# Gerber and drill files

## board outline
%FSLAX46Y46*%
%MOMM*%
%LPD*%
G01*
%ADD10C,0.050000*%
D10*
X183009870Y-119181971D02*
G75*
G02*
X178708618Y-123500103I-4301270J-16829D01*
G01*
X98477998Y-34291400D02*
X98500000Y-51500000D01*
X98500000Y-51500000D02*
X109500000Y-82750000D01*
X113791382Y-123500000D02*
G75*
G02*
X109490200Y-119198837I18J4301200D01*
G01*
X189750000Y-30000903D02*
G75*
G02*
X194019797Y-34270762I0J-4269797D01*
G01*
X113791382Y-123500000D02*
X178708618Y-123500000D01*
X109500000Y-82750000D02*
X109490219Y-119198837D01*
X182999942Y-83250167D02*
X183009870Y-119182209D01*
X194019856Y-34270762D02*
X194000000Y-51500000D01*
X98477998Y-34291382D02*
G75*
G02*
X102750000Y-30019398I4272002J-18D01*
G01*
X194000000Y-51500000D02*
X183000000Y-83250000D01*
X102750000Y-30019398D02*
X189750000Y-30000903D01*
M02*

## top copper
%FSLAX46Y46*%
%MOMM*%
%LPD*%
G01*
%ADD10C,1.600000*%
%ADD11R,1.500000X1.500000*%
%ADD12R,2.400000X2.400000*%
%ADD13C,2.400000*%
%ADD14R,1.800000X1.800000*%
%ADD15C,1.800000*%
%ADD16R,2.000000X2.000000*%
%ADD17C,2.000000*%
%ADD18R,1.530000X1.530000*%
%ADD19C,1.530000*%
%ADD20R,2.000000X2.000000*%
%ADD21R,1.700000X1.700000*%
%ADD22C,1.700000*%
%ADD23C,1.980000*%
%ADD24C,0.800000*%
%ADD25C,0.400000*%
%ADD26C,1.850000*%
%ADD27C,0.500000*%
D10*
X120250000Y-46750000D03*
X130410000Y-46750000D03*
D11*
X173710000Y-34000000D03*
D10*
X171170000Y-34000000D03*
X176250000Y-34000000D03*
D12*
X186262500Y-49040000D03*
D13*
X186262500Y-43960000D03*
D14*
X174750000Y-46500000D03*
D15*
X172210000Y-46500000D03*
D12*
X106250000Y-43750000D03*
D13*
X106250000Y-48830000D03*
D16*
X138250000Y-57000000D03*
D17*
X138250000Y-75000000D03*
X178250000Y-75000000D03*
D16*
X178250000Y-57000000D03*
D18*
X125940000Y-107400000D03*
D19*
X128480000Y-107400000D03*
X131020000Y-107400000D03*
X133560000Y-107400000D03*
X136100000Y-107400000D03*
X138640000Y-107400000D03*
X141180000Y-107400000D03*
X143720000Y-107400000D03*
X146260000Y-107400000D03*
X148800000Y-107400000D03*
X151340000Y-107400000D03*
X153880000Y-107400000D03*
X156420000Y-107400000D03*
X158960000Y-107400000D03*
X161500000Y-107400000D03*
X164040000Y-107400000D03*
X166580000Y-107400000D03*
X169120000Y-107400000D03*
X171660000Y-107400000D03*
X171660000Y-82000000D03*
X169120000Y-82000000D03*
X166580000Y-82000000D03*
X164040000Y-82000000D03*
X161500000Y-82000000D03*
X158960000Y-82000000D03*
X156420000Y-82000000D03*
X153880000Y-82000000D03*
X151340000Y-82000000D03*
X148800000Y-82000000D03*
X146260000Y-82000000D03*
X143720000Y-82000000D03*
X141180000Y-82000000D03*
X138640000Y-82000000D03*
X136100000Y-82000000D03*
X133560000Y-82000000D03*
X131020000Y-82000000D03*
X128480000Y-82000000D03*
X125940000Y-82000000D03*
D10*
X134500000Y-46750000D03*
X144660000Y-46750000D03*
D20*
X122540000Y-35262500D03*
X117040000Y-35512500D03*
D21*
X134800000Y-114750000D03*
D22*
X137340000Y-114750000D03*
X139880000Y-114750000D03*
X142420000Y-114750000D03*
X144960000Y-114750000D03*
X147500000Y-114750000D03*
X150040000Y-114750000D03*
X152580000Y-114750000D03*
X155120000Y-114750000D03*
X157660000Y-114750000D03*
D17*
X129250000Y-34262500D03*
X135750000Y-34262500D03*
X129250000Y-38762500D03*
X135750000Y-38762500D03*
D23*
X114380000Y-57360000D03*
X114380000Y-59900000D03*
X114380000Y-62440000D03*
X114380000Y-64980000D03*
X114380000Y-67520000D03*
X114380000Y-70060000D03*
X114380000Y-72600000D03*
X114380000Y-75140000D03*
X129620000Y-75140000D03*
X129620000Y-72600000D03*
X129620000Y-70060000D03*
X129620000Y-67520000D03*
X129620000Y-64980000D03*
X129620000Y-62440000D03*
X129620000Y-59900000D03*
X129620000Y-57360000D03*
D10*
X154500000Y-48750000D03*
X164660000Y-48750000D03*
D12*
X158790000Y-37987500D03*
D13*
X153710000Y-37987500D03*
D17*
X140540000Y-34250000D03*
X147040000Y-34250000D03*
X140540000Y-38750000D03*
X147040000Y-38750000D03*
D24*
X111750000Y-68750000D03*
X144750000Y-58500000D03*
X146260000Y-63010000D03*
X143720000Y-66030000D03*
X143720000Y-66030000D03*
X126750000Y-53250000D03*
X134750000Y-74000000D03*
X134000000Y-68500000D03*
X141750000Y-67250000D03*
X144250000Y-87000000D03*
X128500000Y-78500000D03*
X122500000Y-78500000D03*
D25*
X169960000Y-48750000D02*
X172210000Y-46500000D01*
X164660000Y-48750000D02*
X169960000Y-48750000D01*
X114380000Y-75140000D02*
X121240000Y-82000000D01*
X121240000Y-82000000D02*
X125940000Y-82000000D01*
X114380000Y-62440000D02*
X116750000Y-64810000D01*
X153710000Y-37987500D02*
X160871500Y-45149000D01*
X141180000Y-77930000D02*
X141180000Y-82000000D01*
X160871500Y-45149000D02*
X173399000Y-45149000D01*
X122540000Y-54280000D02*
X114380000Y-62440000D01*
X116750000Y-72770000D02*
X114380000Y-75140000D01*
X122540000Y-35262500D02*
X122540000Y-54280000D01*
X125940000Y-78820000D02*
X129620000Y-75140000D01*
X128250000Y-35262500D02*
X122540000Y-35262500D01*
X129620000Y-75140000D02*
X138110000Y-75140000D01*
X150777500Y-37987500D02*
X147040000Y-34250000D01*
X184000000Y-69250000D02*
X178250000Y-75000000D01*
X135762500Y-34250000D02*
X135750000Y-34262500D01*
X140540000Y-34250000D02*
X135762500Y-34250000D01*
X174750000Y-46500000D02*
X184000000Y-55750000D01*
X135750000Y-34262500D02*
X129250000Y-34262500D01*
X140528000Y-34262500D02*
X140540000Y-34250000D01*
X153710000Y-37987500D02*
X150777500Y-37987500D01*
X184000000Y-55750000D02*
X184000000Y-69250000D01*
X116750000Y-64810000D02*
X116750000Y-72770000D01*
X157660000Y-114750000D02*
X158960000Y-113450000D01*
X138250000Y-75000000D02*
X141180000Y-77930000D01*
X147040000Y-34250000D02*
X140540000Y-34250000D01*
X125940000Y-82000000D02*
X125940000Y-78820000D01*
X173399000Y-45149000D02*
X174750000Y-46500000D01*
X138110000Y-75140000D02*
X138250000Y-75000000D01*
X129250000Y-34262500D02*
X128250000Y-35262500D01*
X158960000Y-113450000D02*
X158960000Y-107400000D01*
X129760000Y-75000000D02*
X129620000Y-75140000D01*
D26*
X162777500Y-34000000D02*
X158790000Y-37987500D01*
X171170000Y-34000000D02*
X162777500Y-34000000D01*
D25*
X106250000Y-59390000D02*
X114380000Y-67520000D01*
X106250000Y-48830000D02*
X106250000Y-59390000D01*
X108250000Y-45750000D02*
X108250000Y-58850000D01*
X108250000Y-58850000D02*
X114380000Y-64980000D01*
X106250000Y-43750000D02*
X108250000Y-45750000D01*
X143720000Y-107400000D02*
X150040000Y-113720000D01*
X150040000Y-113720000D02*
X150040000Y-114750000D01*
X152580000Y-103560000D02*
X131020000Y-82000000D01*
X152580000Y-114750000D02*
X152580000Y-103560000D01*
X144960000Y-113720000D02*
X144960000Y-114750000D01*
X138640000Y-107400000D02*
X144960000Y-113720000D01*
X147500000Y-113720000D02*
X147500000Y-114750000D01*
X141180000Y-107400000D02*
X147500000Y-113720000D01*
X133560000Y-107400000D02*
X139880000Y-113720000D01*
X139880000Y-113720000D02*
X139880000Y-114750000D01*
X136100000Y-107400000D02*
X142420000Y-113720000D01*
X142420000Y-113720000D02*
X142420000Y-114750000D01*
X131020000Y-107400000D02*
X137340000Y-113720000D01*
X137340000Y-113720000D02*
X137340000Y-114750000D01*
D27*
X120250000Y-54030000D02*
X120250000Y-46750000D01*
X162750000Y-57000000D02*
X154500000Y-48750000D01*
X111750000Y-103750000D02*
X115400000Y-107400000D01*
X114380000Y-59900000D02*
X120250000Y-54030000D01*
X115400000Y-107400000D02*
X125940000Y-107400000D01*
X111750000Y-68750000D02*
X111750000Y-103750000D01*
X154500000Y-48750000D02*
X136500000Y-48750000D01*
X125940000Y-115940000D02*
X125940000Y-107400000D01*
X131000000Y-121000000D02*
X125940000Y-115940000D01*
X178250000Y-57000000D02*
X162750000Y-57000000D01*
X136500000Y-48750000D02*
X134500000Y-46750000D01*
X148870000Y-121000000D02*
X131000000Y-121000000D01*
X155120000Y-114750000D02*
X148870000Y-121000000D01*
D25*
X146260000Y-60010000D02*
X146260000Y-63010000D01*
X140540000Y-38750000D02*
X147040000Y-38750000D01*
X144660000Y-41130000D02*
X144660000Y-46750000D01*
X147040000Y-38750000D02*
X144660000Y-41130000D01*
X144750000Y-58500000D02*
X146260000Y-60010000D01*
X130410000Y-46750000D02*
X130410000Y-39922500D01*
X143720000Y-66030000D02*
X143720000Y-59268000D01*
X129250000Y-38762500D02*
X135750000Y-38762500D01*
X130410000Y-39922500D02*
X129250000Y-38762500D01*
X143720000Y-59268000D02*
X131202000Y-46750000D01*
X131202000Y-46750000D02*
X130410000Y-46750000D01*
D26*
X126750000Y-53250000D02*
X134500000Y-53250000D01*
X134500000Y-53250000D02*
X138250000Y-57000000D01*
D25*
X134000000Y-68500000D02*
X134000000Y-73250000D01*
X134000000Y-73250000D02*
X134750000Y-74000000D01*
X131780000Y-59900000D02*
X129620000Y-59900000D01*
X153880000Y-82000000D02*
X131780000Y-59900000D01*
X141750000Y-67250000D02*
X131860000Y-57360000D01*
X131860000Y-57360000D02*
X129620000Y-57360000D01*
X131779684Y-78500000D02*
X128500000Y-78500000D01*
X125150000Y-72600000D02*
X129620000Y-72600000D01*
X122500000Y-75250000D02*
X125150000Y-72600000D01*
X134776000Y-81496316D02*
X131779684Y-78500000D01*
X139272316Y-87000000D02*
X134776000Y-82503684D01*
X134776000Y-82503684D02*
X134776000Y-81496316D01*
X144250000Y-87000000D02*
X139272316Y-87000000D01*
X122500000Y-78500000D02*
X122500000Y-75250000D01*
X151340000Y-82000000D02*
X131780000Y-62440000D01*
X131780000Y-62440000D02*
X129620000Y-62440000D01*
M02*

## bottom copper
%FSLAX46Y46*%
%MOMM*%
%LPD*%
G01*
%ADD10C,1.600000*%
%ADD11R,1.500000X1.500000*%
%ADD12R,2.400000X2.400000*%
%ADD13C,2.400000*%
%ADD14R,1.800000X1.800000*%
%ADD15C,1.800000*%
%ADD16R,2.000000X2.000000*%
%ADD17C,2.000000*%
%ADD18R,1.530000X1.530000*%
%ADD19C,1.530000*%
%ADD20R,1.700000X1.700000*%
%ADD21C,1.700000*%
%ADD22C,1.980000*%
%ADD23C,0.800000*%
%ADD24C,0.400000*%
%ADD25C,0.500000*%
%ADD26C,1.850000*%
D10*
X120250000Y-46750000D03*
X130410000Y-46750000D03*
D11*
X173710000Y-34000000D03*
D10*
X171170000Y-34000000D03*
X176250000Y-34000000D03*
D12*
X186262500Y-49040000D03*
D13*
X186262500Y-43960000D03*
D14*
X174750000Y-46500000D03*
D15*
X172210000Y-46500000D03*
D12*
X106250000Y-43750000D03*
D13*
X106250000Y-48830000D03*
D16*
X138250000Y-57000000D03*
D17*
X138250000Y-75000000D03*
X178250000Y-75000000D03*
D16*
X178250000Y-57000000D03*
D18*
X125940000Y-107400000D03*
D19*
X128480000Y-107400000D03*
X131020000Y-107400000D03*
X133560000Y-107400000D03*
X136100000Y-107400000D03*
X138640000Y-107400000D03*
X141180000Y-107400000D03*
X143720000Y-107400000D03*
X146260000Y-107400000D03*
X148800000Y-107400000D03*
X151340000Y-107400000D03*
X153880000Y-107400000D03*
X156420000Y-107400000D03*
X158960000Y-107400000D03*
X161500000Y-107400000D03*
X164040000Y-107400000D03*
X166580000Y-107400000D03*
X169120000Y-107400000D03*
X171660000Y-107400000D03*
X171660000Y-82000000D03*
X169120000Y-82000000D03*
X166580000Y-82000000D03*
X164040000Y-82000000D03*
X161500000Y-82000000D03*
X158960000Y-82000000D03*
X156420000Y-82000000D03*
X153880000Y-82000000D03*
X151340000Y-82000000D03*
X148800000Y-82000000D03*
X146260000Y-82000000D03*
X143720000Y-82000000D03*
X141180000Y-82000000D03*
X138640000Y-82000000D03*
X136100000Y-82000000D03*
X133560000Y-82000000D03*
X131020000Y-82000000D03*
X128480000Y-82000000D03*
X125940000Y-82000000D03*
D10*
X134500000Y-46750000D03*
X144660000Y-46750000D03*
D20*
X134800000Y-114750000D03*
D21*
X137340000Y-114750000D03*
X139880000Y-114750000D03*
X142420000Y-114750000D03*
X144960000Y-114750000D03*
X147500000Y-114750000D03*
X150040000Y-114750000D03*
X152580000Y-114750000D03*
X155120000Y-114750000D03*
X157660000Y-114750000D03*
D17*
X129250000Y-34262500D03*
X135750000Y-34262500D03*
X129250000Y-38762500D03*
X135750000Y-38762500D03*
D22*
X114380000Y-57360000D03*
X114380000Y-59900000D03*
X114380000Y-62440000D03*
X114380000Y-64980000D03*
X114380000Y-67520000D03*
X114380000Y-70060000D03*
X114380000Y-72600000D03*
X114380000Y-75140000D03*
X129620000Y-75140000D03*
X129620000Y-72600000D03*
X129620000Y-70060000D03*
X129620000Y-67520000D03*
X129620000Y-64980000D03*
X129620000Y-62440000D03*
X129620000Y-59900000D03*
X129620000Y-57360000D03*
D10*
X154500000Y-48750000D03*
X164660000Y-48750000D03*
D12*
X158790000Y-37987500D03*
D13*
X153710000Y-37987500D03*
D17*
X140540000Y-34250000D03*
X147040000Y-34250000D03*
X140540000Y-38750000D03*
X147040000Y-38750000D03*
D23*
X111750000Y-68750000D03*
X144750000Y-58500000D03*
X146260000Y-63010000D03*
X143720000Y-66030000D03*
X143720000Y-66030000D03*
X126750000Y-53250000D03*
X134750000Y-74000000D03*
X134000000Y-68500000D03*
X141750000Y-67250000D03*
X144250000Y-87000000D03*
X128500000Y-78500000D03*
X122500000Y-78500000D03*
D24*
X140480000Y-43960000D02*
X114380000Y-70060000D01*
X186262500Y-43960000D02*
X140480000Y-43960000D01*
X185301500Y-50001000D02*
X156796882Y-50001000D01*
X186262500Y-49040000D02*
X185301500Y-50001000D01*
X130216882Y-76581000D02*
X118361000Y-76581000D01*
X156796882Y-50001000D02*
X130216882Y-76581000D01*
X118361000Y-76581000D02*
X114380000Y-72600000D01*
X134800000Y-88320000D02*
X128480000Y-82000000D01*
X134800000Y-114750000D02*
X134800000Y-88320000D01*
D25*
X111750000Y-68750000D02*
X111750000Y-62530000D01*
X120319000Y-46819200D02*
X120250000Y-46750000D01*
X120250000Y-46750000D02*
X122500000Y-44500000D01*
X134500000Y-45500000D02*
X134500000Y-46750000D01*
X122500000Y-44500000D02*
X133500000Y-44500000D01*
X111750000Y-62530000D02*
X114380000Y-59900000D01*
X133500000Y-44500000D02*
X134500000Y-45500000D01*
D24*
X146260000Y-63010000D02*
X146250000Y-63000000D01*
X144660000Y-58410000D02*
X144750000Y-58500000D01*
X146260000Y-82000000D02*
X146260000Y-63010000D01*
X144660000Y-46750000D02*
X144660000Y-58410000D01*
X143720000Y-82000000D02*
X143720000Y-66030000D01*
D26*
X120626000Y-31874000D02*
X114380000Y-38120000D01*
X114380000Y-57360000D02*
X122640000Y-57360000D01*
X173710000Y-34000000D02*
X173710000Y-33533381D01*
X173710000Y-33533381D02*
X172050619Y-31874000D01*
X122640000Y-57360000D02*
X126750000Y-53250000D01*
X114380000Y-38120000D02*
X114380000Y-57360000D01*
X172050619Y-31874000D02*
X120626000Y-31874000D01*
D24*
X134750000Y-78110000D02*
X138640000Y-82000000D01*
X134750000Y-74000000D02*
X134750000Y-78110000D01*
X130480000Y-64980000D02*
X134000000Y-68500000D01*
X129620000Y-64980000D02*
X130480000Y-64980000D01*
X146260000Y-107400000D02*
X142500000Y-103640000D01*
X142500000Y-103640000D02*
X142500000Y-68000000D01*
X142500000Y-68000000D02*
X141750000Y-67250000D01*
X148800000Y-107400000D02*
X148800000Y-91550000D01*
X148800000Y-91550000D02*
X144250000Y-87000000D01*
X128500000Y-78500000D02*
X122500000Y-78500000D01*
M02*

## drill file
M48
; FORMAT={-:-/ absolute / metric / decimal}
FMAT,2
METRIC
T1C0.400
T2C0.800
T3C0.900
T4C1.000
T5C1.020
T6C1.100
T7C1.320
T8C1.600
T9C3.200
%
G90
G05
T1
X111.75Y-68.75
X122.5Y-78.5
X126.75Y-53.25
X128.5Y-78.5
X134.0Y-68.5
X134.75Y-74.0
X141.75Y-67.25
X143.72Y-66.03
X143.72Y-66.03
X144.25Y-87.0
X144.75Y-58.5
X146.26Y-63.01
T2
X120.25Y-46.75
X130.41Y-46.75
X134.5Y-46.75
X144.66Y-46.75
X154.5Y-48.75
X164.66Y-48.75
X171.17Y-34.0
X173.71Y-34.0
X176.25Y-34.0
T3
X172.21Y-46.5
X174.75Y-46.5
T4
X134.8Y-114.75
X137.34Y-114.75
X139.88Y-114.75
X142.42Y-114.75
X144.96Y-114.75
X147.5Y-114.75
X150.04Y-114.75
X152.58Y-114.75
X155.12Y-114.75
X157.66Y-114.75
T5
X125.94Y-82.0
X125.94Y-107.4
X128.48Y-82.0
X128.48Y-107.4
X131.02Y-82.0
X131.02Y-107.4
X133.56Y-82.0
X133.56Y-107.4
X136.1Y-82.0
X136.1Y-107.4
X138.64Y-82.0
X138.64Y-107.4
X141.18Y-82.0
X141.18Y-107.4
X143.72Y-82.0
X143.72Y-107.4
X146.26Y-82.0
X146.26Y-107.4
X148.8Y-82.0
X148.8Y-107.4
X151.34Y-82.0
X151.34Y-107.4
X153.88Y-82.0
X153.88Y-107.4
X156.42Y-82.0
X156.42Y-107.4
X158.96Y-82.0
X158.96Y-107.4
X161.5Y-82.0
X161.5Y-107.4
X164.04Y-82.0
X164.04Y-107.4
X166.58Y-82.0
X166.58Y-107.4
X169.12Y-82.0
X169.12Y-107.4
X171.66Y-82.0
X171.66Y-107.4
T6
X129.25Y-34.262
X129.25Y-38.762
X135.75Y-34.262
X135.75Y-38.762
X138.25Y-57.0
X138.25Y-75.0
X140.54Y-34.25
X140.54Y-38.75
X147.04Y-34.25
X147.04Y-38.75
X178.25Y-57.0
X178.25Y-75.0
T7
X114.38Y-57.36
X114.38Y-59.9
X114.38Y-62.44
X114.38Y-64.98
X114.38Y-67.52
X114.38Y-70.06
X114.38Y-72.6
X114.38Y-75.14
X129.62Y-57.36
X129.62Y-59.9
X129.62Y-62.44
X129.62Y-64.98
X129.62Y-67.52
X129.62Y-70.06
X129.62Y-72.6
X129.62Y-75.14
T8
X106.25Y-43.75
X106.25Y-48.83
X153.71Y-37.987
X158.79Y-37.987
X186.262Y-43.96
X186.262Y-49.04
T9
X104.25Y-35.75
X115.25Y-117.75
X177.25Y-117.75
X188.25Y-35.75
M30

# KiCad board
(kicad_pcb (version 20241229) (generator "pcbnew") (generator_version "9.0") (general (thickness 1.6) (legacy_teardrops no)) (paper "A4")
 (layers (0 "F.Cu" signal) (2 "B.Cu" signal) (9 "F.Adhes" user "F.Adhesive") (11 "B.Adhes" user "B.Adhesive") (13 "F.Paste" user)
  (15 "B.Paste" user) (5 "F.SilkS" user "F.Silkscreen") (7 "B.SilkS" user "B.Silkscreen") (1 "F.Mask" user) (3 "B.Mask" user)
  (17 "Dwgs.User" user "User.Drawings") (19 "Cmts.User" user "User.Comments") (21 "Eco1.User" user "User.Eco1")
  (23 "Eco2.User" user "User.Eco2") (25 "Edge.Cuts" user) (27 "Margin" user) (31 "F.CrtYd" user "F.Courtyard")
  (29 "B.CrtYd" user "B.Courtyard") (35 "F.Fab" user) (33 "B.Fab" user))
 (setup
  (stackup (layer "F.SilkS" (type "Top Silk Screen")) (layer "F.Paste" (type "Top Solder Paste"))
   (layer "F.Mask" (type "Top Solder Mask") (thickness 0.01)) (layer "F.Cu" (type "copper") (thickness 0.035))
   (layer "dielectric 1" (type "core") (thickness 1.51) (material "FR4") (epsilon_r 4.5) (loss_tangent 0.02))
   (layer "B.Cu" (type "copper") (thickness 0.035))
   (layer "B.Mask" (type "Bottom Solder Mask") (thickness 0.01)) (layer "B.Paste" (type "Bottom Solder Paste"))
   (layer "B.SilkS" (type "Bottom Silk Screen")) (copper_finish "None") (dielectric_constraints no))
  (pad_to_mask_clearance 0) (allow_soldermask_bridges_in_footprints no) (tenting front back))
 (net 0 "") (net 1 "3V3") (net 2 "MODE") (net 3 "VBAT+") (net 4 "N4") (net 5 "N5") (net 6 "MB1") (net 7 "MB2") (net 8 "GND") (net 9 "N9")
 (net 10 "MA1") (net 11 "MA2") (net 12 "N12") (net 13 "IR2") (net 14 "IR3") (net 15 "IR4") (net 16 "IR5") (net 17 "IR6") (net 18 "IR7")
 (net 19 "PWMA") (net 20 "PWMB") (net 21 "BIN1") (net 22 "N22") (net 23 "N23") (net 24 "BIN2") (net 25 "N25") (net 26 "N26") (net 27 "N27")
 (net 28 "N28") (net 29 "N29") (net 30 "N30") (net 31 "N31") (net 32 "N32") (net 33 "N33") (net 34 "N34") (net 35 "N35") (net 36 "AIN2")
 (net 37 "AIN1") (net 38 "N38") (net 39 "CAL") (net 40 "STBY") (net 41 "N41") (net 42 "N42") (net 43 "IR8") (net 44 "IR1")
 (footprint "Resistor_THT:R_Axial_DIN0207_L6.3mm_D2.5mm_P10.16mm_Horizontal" (layer "F.Cu") (at 120.25 46.75)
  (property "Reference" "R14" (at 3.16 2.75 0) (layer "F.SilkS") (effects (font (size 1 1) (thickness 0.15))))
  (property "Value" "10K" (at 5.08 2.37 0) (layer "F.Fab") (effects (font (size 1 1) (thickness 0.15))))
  (pad "1" thru_hole circle (at 0 0) (size 1.6 1.6) (drill 0.8) (layers "*.Cu" "*.Mask") (remove_unused_layers no) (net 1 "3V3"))
  (pad "2" thru_hole circle (at 10.16 0) (size 1.6 1.6) (drill 0.8) (layers "*.Cu" "*.Mask") (remove_unused_layers no) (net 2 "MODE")))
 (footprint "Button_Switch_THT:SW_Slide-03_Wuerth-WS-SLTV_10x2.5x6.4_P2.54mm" (layer "F.Cu") (at 173.71 34)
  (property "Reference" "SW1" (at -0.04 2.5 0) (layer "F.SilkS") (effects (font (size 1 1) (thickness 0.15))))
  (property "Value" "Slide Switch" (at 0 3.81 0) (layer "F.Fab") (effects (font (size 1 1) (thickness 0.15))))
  (pad "1" thru_hole rect (at 0 0) (size 1.5 1.5) (drill 0.8) (layers "*.Cu" "*.Mask") (remove_unused_layers no) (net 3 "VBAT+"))
  (pad "2" thru_hole circle (at -2.54 0) (size 1.6 1.6) (drill 0.8) (layers "*.Cu" "*.Mask") (remove_unused_layers no) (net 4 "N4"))
  (pad "3" thru_hole circle (at 2.54 0) (size 1.6 1.6) (drill 0.8) (layers "*.Cu" "*.Mask") (remove_unused_layers no) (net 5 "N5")))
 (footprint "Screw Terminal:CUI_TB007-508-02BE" (layer "F.Cu") (at 186.2625 49.04 90)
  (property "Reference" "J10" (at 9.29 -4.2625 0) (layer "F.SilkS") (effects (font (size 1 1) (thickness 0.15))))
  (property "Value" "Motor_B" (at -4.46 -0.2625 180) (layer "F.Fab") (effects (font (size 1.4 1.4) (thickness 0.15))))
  (pad "1" thru_hole rect (at 0 0 90) (size 2.4 2.4) (drill 1.6) (layers "*.Cu" "*.Mask") (remove_unused_layers no) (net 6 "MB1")
   (solder_mask_margin 0.102))
  (pad "2" thru_hole circle (at 5.08 0 90) (size 2.4 2.4) (drill 1.6) (layers "*.Cu" "*.Mask") (remove_unused_layers no) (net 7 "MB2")
   (solder_mask_margin 0.102)))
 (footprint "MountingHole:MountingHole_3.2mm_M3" (layer "F.Cu") (at 177.25 117.75)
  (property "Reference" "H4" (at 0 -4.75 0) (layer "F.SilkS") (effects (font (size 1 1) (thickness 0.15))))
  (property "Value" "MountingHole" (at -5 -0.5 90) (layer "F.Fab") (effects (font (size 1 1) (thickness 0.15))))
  (pad "" np_thru_hole circle (at 0 0) (size 3.2 3.2) (drill 3.2) (layers "*.Cu" "*.Mask")))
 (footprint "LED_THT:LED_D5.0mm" (layer "F.Cu") (at 174.75 46.5 180)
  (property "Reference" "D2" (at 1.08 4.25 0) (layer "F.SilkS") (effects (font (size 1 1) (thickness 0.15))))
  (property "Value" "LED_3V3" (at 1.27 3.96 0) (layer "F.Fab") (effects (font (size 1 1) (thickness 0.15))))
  (pad "1" thru_hole rect (at 0 0 180) (size 1.8 1.8) (drill 0.9) (layers "*.Cu" "*.Mask") (remove_unused_layers no) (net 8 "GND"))
  (pad "2" thru_hole circle (at 2.54 0 180) (size 1.8 1.8) (drill 0.9) (layers "*.Cu" "*.Mask") (remove_unused_layers no) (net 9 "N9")))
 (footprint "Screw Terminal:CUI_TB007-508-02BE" (layer "F.Cu") (at 106.25 43.75 -90)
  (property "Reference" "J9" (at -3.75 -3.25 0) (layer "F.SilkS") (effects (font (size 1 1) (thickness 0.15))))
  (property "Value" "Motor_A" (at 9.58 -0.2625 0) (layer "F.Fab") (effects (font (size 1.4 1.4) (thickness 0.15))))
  (pad "1" thru_hole rect (at 0 0 270) (size 2.4 2.4) (drill 1.6) (layers "*.Cu" "*.Mask") (remove_unused_layers no) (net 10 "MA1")
   (solder_mask_margin 0.102))
  (pad "2" thru_hole circle (at 5.08 0 270) (size 2.4 2.4) (drill 1.6) (layers "*.Cu" "*.Mask") (remove_unused_layers no) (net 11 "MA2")
   (solder_mask_margin 0.102)))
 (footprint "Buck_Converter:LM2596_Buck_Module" (layer "F.Cu") (at 136.85 76.4)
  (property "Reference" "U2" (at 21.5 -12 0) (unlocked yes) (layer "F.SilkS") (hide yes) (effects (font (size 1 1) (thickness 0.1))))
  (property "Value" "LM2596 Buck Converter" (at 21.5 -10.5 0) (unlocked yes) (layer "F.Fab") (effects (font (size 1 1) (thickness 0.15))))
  (pad "1" thru_hole rect (at 1.4 -19.4) (size 2 2) (drill 1.1) (layers "*.Cu" "*.Mask") (remove_unused_layers no) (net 3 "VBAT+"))
  (pad "2" thru_hole circle (at 1.4 -1.4) (size 2 2) (drill 1.1) (layers "*.Cu" "*.Mask") (remove_unused_layers no) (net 8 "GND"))
  (pad "3" thru_hole circle (at 41.4 -1.4) (size 2 2) (drill 1.1) (layers "*.Cu" "*.Mask") (remove_unused_layers no) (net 8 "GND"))
  (pad "4" thru_hole rect (at 41.4 -19.4) (size 2 2) (drill 1.1) (layers "*.Cu" "*.Mask") (remove_unused_layers no) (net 1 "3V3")))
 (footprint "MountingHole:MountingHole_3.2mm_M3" (layer "F.Cu") (at 115.25 117.75)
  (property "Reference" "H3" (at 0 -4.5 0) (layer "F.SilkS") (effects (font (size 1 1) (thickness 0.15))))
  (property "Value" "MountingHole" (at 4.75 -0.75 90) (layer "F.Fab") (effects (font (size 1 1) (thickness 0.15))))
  (pad "" np_thru_hole circle (at 0 0) (size 3.2 3.2) (drill 3.2) (layers "*.Cu" "*.Mask")))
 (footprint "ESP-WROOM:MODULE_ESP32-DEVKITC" (layer "F.Cu") (at 148.79 94.7 90)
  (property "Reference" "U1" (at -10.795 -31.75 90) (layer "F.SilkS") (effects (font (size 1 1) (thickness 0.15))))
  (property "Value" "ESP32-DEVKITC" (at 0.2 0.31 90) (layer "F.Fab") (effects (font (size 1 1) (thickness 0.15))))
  (pad "1" thru_hole rect (at -12.7 -22.85 90) (size 1.53 1.53) (drill 1.02) (layers "*.Cu" "*.Mask") (remove_unused_layers no)
   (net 1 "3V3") (solder_mask_margin 0.102))
  (pad "2" thru_hole circle (at -12.7 -20.31 90) (size 1.53 1.53) (drill 1.02) (layers "*.Cu" "*.Mask") (remove_unused_layers no)
   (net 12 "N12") (solder_mask_margin 0.102))
  (pad "3" thru_hole circle (at -12.7 -17.77 90) (size 1.53 1.53) (drill 1.02) (layers "*.Cu" "*.Mask") (remove_unused_layers no)
   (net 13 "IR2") (solder_mask_margin 0.102))
  (pad "4" thru_hole circle (at -12.7 -15.23 90) (size 1.53 1.53) (drill 1.02) (layers "*.Cu" "*.Mask") (remove_unused_layers no)
   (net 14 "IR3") (solder_mask_margin 0.102))
  (pad "5" thru_hole circle (at -12.7 -12.69 90) (size 1.53 1.53) (drill 1.02) (layers "*.Cu" "*.Mask") (remove_unused_layers no)
   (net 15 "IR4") (solder_mask_margin 0.102))
  (pad "6" thru_hole circle (at -12.7 -10.15 90) (size 1.53 1.53) (drill 1.02) (layers "*.Cu" "*.Mask") (remove_unused_layers no)
   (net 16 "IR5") (solder_mask_margin 0.102))
  (pad "7" thru_hole circle (at -12.7 -7.61 90) (size 1.53 1.53) (drill 1.02) (layers "*.Cu" "*.Mask") (remove_unused_layers no)
   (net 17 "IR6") (solder_mask_margin 0.102))
  (pad "8" thru_hole circle (at -12.7 -5.07 90) (size 1.53 1.53) (drill 1.02) (layers "*.Cu" "*.Mask") (remove_unused_layers no)
   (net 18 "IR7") (solder_mask_margin 0.102))
  (pad "9" thru_hole circle (at -12.7 -2.53 90) (size 1.53 1.53) (drill 1.02) (layers "*.Cu" "*.Mask") (remove_unused_layers no)
   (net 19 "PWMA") (solder_mask_margin 0.102))
  (pad "10" thru_hole circle (at -12.7 0.01 90) (size 1.53 1.53) (drill 1.02) (layers "*.Cu" "*.Mask") (remove_unused_layers no)
   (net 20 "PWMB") (solder_mask_margin 0.102))
  (pad "11" thru_hole circle (at -12.7 2.55 90) (size 1.53 1.53) (drill 1.02) (layers "*.Cu" "*.Mask") (remove_unused_layers no)
   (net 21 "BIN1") (solder_mask_margin 0.102))
  (pad "12" thru_hole circle (at -12.7 5.09 90) (size 1.53 1.53) (drill 1.02) (layers "*.Cu" "*.Mask") (remove_unused_layers no)
   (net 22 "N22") (solder_mask_margin 0.102))
  (pad "13" thru_hole circle (at -12.7 7.63 90) (size 1.53 1.53) (drill 1.02) (layers "*.Cu" "*.Mask") (remove_unused_layers no)
   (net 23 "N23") (solder_mask_margin 0.102))
  (pad "14" thru_hole circle (at -12.7 10.17 90) (size 1.53 1.53) (drill 1.02) (layers "*.Cu" "*.Mask") (remove_unused_layers no)
   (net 8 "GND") (solder_mask_margin 0.102))
  (pad "15" thru_hole circle (at -12.7 12.71 90) (size 1.53 1.53) (drill 1.02) (layers "*.Cu" "*.Mask") (remove_unused_layers no)
   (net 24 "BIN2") (solder_mask_margin 0.102))
  (pad "16" thru_hole circle (at -12.7 15.25 90) (size 1.53 1.53) (drill 1.02) (layers "*.Cu" "*.Mask") (remove_unused_layers no)
   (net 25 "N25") (solder_mask_margin 0.102))
  (pad "17" thru_hole circle (at -12.7 17.79 90) (size 1.53 1.53) (drill 1.02) (layers "*.Cu" "*.Mask") (remove_unused_layers no)
   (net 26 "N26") (solder_mask_margin 0.102))
  (pad "18" thru_hole circle (at -12.7 20.33 90) (size 1.53 1.53) (drill 1.02) (layers "*.Cu" "*.Mask") (remove_unused_layers no)
   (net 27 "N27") (solder_mask_margin 0.102))
  (pad "19" thru_hole circle (at -12.7 22.87 90) (size 1.53 1.53) (drill 1.02) (layers "*.Cu" "*.Mask") (remove_unused_layers no)
   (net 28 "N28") (solder_mask_margin 0.102))
  (pad "20" thru_hole circle (at 12.7 22.87 90) (size 1.53 1.53) (drill 1.02) (layers "*.Cu" "*.Mask") (remove_unused_layers no)
   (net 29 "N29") (solder_mask_margin 0.102))
  (pad "21" thru_hole circle (at 12.7 20.33 90) (size 1.53 1.53) (drill 1.02) (layers "*.Cu" "*.Mask") (remove_unused_layers no)
   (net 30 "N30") (solder_mask_margin 0.102))
  (pad "22" thru_hole circle (at 12.7 17.79 90) (size 1.53 1.53) (drill 1.02) (layers "*.Cu" "*.Mask") (remove_unused_layers no)
   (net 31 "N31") (solder_mask_margin 0.102))
  (pad "23" thru_hole circle (at 12.7 15.25 90) (size 1.53 1.53) (drill 1.02) (layers "*.Cu" "*.Mask") (remove_unused_layers no)
   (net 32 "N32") (solder_mask_margin 0.102))
  (pad "24" thru_hole circle (at 12.7 12.71 90) (size 1.53 1.53) (drill 1.02) (layers "*.Cu" "*.Mask") (remove_unused_layers no)
   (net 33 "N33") (solder_mask_margin 0.102))
  (pad "25" thru_hole circle (at 12.7 10.17 90) (size 1.53 1.53) (drill 1.02) (layers "*.Cu" "*.Mask") (remove_unused_layers no)
   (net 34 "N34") (solder_mask_margin 0.102))
  (pad "26" thru_hole circle (at 12.7 7.63 90) (size 1.53 1.53) (drill 1.02) (layers "*.Cu" "*.Mask") (remove_unused_layers no)
   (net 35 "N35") (solder_mask_margin 0.102))
  (pad "27" thru_hole circle (at 12.7 5.09 90) (size 1.53 1.53) (drill 1.02) (layers "*.Cu" "*.Mask") (remove_unused_layers no)
   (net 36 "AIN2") (solder_mask_margin 0.102))
  (pad "28" thru_hole circle (at 12.7 2.55 90) (size 1.53 1.53) (drill 1.02) (layers "*.Cu" "*.Mask") (remove_unused_layers no)
   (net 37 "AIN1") (solder_mask_margin 0.102))
  (pad "29" thru_hole circle (at 12.7 0.01 90) (size 1.53 1.53) (drill 1.02) (layers "*.Cu" "*.Mask") (remove_unused_layers no)
   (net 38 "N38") (solder_mask_margin 0.102))
  (pad "30" thru_hole circle (at 12.7 -2.53 90) (size 1.53 1.53) (drill 1.02) (layers "*.Cu" "*.Mask") (remove_unused_layers no)
   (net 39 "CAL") (solder_mask_margin 0.102))
  (pad "31" thru_hole circle (at 12.7 -5.07 90) (size 1.53 1.53) (drill 1.02) (layers "*.Cu" "*.Mask") (remove_unused_layers no)
   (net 2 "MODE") (solder_mask_margin 0.102))
  (pad "32" thru_hole circle (at 12.7 -7.61 90) (size 1.53 1.53) (drill 1.02) (layers "*.Cu" "*.Mask") (remove_unused_layers no)
   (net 8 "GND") (solder_mask_margin 0.102))
  (pad "33" thru_hole circle (at 12.7 -10.15 90) (size 1.53 1.53) (drill 1.02) (layers "*.Cu" "*.Mask") (remove_unused_layers no)
   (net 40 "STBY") (solder_mask_margin 0.102))
  (pad "34" thru_hole circle (at 12.7 -12.69 90) (size 1.53 1.53) (drill 1.02) (layers "*.Cu" "*.Mask") (remove_unused_layers no)
   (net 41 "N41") (solder_mask_margin 0.102))
  (pad "35" thru_hole circle (at 12.7 -15.23 90) (size 1.53 1.53) (drill 1.02) (layers "*.Cu" "*.Mask") (remove_unused_layers no)
   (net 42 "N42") (solder_mask_margin 0.102))
  (pad "36" thru_hole circle (at 12.7 -17.77 90) (size 1.53 1.53) (drill 1.02) (layers "*.Cu" "*.Mask") (remove_unused_layers no)
   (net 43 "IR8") (solder_mask_margin 0.102))
  (pad "37" thru_hole circle (at 12.7 -20.31 90) (size 1.53 1.53) (drill 1.02) (layers "*.Cu" "*.Mask") (remove_unused_layers no)
   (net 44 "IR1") (solder_mask_margin 0.102))
  (pad "38" thru_hole circle (at 12.7 -22.85 90) (size 1.53 1.53) (drill 1.02) (layers "*.Cu" "*.Mask") (remove_unused_layers no)
   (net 8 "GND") (solder_mask_margin 0.102)))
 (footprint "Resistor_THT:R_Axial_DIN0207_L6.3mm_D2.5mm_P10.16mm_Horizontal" (layer "F.Cu") (at 134.5 46.75)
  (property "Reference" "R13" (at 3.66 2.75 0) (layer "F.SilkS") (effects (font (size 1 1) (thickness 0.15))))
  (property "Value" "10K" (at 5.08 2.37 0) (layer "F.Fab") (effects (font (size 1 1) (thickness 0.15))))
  (pad "1" thru_hole circle (at 0 0) (size 1.6 1.6) (drill 0.8) (layers "*.Cu" "*.Mask") (remove_unused_layers no) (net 1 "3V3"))
  (pad "2" thru_hole circle (at 10.16 0) (size 1.6 1.6) (drill 0.8) (layers "*.Cu" "*.Mask") (remove_unused_layers no) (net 39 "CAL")))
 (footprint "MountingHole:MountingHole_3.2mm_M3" (layer "F.Cu") (at 188.25 35.75)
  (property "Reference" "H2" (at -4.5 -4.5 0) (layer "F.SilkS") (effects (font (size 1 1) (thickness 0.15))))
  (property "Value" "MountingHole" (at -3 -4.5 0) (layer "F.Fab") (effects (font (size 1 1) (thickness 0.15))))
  (pad "" np_thru_hole circle (at 0 0) (size 3.2 3.2) (drill 3.2) (layers "*.Cu" "*.Mask")))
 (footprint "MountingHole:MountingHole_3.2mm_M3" (layer "F.Cu") (at 104.25 35.75)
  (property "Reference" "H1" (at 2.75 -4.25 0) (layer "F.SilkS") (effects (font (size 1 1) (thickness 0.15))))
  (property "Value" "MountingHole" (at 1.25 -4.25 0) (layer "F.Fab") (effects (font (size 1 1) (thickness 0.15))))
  (pad "" np_thru_hole circle (at 0 0) (size 3.2 3.2) (drill 3.2) (layers "*.Cu" "*.Mask")))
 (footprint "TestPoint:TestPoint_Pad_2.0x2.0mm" (layer "F.Cu") (at 122.54 35.2625)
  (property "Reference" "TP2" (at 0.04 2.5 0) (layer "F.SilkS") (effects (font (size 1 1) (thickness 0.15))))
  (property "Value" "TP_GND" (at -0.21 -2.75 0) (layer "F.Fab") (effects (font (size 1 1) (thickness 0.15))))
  (pad "1" smd rect (at 0 0) (size 2 2) (layers "F.Cu" "F.Mask") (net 8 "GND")))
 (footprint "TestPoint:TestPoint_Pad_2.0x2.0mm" (layer "F.Cu") (at 117.04 35.5125 180)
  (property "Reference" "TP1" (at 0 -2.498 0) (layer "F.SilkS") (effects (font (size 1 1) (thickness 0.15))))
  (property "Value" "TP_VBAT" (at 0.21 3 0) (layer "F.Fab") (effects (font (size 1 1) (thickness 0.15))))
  (pad "1" smd rect (at 0 0 180) (size 2 2) (layers "F.Cu" "F.Mask") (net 3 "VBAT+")))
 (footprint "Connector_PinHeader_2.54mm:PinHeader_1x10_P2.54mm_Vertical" (layer "F.Cu") (at 134.8 114.75 90)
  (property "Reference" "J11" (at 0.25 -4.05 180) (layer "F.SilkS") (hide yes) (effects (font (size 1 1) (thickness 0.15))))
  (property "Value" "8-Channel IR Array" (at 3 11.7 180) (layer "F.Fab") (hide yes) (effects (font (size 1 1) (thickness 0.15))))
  (pad "1" thru_hole rect (at 0 0 90) (size 1.7 1.7) (drill 1) (layers "*.Cu" "*.Mask") (remove_unused_layers no) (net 44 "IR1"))
  (pad "2" thru_hole circle (at 0 2.54 90) (size 1.7 1.7) (drill 1) (layers "*.Cu" "*.Mask") (remove_unused_layers no) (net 13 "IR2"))
  (pad "3" thru_hole circle (at 0 5.08 90) (size 1.7 1.7) (drill 1) (layers "*.Cu" "*.Mask") (remove_unused_layers no) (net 14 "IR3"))
  (pad "4" thru_hole circle (at 0 7.62 90) (size 1.7 1.7) (drill 1) (layers "*.Cu" "*.Mask") (remove_unused_layers no) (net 15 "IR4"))
  (pad "5" thru_hole circle (at 0 10.16 90) (size 1.7 1.7) (drill 1) (layers "*.Cu" "*.Mask") (remove_unused_layers no) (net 16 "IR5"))
  (pad "6" thru_hole circle (at 0 12.7 90) (size 1.7 1.7) (drill 1) (layers "*.Cu" "*.Mask") (remove_unused_layers no) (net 17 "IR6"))
  (pad "7" thru_hole circle (at 0 15.24 90) (size 1.7 1.7) (drill 1) (layers "*.Cu" "*.Mask") (remove_unused_layers no) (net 18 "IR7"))
  (pad "8" thru_hole circle (at 0 17.78 90) (size 1.7 1.7) (drill 1) (layers "*.Cu" "*.Mask") (remove_unused_layers no) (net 43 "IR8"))
  (pad "9" thru_hole circle (at 0 20.32 90) (size 1.7 1.7) (drill 1) (layers "*.Cu" "*.Mask") (remove_unused_layers no) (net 1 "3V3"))
  (pad "10" thru_hole circle (at 0 22.86 90) (size 1.7 1.7) (drill 1) (layers "*.Cu" "*.Mask") (remove_unused_layers no) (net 8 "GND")))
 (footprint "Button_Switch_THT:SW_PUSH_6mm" (layer "F.Cu") (at 129.25 34.2625)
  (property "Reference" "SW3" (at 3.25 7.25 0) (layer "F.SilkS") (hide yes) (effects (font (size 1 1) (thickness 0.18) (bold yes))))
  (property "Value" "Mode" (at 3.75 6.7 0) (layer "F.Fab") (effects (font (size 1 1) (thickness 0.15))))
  (pad "1" thru_hole circle (at 0 0 90) (size 2 2) (drill 1.1) (layers "*.Cu" "*.Mask") (remove_unused_layers no) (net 8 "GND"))
  (pad "1" thru_hole circle (at 6.5 0 90) (size 2 2) (drill 1.1) (layers "*.Cu" "*.Mask") (remove_unused_layers no) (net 8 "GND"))
  (pad "2" thru_hole circle (at 0 4.5 90) (size 2 2) (drill 1.1) (layers "*.Cu" "*.Mask") (remove_unused_layers no) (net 2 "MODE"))
  (pad "2" thru_hole circle (at 6.5 4.5 90) (size 2 2) (drill 1.1) (layers "*.Cu" "*.Mask") (remove_unused_layers no) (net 2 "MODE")))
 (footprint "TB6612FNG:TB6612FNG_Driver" (layer "F.Cu") (at 122 66.25)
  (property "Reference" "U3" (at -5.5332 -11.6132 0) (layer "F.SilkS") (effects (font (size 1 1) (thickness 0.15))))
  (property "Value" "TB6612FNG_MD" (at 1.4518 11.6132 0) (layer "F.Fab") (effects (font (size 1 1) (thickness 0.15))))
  (pad "1" thru_hole circle (at -7.62 -8.89) (size 1.98 1.98) (drill 1.32) (layers "*.Cu" "*.Mask") (remove_unused_layers no)
   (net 3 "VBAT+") (solder_mask_margin 0.102))
  (pad "2" thru_hole circle (at -7.62 -6.35) (size 1.98 1.98) (drill 1.32) (layers "*.Cu" "*.Mask") (remove_unused_layers no) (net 1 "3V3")
   (solder_mask_margin 0.102))
  (pad "3" thru_hole circle (at -7.62 -3.81) (size 1.98 1.98) (drill 1.32) (layers "*.Cu" "*.Mask") (remove_unused_layers no) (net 8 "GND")
   (solder_mask_margin 0.102))
  (pad "4" thru_hole circle (at -7.62 -1.27) (size 1.98 1.98) (drill 1.32) (layers "*.Cu" "*.Mask") (remove_unused_layers no) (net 10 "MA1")
   (solder_mask_margin 0.102))
  (pad "5" thru_hole circle (at -7.62 1.27) (size 1.98 1.98) (drill 1.32) (layers "*.Cu" "*.Mask") (remove_unused_layers no) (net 11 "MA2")
   (solder_mask_margin 0.102))
  (pad "6" thru_hole circle (at -7.62 3.81) (size 1.98 1.98) (drill 1.32) (layers "*.Cu" "*.Mask") (remove_unused_layers no) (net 7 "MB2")
   (solder_mask_margin 0.102))
  (pad "7" thru_hole circle (at -7.62 6.35) (size 1.98 1.98) (drill 1.32) (layers "*.Cu" "*.Mask") (remove_unused_layers no) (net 6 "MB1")
   (solder_mask_margin 0.102))
  (pad "8" thru_hole circle (at -7.62 8.89) (size 1.98 1.98) (drill 1.32) (layers "*.Cu" "*.Mask") (remove_unused_layers no) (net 8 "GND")
   (solder_mask_margin 0.102))
  (pad "9" thru_hole circle (at 7.62 8.89) (size 1.98 1.98) (drill 1.32) (layers "*.Cu" "*.Mask") (remove_unused_layers no) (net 8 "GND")
   (solder_mask_margin 0.102))
  (pad "10" thru_hole circle (at 7.62 6.35) (size 1.98 1.98) (drill 1.32) (layers "*.Cu" "*.Mask") (remove_unused_layers no) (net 20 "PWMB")
   (solder_mask_margin 0.102))
  (pad "11" thru_hole circle (at 7.62 3.81) (size 1.98 1.98) (drill 1.32) (layers "*.Cu" "*.Mask") (remove_unused_layers no) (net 24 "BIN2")
   (solder_mask_margin 0.102))
  (pad "12" thru_hole circle (at 7.62 1.27) (size 1.98 1.98) (drill 1.32) (layers "*.Cu" "*.Mask") (remove_unused_layers no) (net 21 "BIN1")
   (solder_mask_margin 0.102))
  (pad "13" thru_hole circle (at 7.62 -1.27) (size 1.98 1.98) (drill 1.32) (layers "*.Cu" "*.Mask") (remove_unused_layers no)
   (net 40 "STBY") (solder_mask_margin 0.102))
  (pad "14" thru_hole circle (at 7.62 -3.81) (size 1.98 1.98) (drill 1.32) (layers "*.Cu" "*.Mask") (remove_unused_layers no)
   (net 37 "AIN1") (solder_mask_margin 0.102))
  (pad "15" thru_hole circle (at 7.62 -6.35) (size 1.98 1.98) (drill 1.32) (layers "*.Cu" "*.Mask") (remove_unused_layers no)
   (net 36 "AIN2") (solder_mask_margin 0.102))
  (pad "16" thru_hole circle (at 7.62 -8.89) (size 1.98 1.98) (drill 1.32) (layers "*.Cu" "*.Mask") (remove_unused_layers no)
   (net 19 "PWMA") (solder_mask_margin 0.102)))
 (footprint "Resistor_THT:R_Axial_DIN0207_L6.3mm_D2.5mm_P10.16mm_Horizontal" (layer "F.Cu") (at 154.5 48.75)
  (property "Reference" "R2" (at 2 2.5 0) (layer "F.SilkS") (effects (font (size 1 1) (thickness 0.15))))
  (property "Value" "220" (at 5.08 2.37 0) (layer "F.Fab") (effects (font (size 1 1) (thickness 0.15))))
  (pad "1" thru_hole circle (at 0 0) (size 1.6 1.6) (drill 0.8) (layers "*.Cu" "*.Mask") (remove_unused_layers no) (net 1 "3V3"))
  (pad "2" thru_hole circle (at 10.16 0) (size 1.6 1.6) (drill 0.8) (layers "*.Cu" "*.Mask") (remove_unused_layers no) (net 9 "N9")))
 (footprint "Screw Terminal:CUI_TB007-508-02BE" (layer "F.Cu") (at 158.79 37.9875 180)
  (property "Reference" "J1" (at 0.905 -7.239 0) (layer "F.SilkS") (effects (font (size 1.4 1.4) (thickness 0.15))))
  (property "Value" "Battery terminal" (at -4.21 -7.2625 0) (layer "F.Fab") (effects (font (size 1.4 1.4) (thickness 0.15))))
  (pad "1" thru_hole rect (at 0 0 180) (size 2.4 2.4) (drill 1.6) (layers "*.Cu" "*.Mask") (remove_unused_layers no) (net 4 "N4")
   (solder_mask_margin 0.102))
  (pad "2" thru_hole circle (at 5.08 0 180) (size 2.4 2.4) (drill 1.6) (layers "*.Cu" "*.Mask") (remove_unused_layers no) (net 8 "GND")
   (solder_mask_margin 0.102)))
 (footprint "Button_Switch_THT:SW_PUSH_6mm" (layer "F.Cu") (at 140.54 34.25)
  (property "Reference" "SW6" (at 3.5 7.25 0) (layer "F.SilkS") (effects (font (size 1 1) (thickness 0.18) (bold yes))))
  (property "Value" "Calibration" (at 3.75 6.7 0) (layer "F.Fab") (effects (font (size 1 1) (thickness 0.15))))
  (pad "1" thru_hole circle (at 0 0 90) (size 2 2) (drill 1.1) (layers "*.Cu" "*.Mask") (remove_unused_layers no) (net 8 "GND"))
  (pad "1" thru_hole circle (at 6.5 0 90) (size 2 2) (drill 1.1) (layers "*.Cu" "*.Mask") (remove_unused_layers no) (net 8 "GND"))
  (pad "2" thru_hole circle (at 0 4.5 90) (size 2 2) (drill 1.1) (layers "*.Cu" "*.Mask") (remove_unused_layers no) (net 39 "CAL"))
  (pad "2" thru_hole circle (at 6.5 4.5 90) (size 2 2) (drill 1.1) (layers "*.Cu" "*.Mask") (remove_unused_layers no) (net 39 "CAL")))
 (gr_arc (start 183.00987 119.181971) (mid 181.756043 122.234336) (end 178.708618 123.500122) (stroke (width 0.05) (type default))
  (layer "Edge.Cuts"))
 (gr_line (start 98.477998 34.2914) (end 98.5 51.5) (stroke (width 0.05) (type default)) (layer "Edge.Cuts"))
 (gr_line (start 98.5 51.5) (end 109.5 82.75) (stroke (width 0.05) (type default)) (layer "Edge.Cuts"))
 (gr_arc (start 113.791382 123.5) (mid 110.75 122.240219) (end 109.490219 119.198837) (stroke (width 0.05) (type default))
  (layer "Edge.Cuts"))
 (gr_arc (start 189.75 30.000903) (mid 192.76926 31.251513) (end 194.019859 34.270762) (stroke (width 0.05) (type default))
  (layer "Edge.Cuts"))
 (gr_line (start 113.791382 123.5) (end 178.708618 123.5) (stroke (width 0.05) (type default)) (layer "Edge.Cuts"))
 (gr_line (start 109.5 82.75) (end 109.490219 119.198837) (stroke (width 0.05) (type default)) (layer "Edge.Cuts"))
 (gr_line (start 182.999942 83.250167) (end 183.00987 119.182209) (stroke (width 0.05) (type default)) (layer "Edge.Cuts"))
 (gr_line (start 194.019856 34.270762) (end 194 51.5) (stroke (width 0.05) (type default)) (layer "Edge.Cuts"))
 (gr_arc (start 98.477998 34.291382) (mid 99.729245 31.270632) (end 102.75 30.01938) (stroke (width 0.05) (type default))
  (layer "Edge.Cuts"))
 (gr_line (start 194 51.5) (end 183 83.25) (stroke (width 0.05) (type default)) (layer "Edge.Cuts"))
 (gr_line (start 102.75 30.019398) (end 189.75 30.000903) (stroke (width 0.05) (type default)) (layer "Edge.Cuts"))
 (segment (start 169.96 48.75) (end 172.21 46.5) (width 0.4) (layer "F.Cu") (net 9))
 (segment (start 164.66 48.75) (end 169.96 48.75) (width 0.4) (layer "F.Cu") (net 9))
 (segment (start 114.38 75.14) (end 121.24 82) (width 0.4) (layer "F.Cu") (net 8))
 (segment (start 121.24 82) (end 125.94 82) (width 0.4) (layer "F.Cu") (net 8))
 (segment (start 114.38 62.44) (end 116.75 64.81) (width 0.4) (layer "F.Cu") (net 8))
 (segment (start 153.71 37.9875) (end 160.8715 45.149) (width 0.4) (layer "F.Cu") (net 8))
 (segment (start 141.18 77.93) (end 141.18 82) (width 0.4) (layer "F.Cu") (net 8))
 (segment (start 160.8715 45.149) (end 173.399 45.149) (width 0.4) (layer "F.Cu") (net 8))
 (segment (start 122.54 54.28) (end 114.38 62.44) (width 0.4) (layer "F.Cu") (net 8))
 (segment (start 116.75 72.77) (end 114.38 75.14) (width 0.4) (layer "F.Cu") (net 8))
 (segment (start 122.54 35.2625) (end 122.54 54.28) (width 0.4) (layer "F.Cu") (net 8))
 (segment (start 125.94 78.82) (end 129.62 75.14) (width 0.4) (layer "F.Cu") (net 8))
 (segment (start 128.25 35.2625) (end 122.54 35.2625) (width 0.4) (layer "F.Cu") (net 8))
 (segment (start 129.62 75.14) (end 138.11 75.14) (width 0.4) (layer "F.Cu") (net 8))
 (segment (start 150.7775 37.9875) (end 147.04 34.25) (width 0.4) (layer "F.Cu") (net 8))
 (segment (start 184 69.25) (end 178.25 75) (width 0.4) (layer "F.Cu") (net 8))
 (segment (start 135.7625 34.25) (end 135.75 34.2625) (width 0.4) (layer "F.Cu") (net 8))
 (segment (start 140.54 34.25) (end 135.7625 34.25) (width 0.4) (layer "F.Cu") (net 8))
 (segment (start 174.75 46.5) (end 184 55.75) (width 0.4) (layer "F.Cu") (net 8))
 (segment (start 135.75 34.2625) (end 129.25 34.2625) (width 0.4) (layer "F.Cu") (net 8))
 (segment (start 140.528 34.2625) (end 140.54 34.25) (width 0.4) (layer "F.Cu") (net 8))
 (segment (start 153.71 37.9875) (end 150.7775 37.9875) (width 0.4) (layer "F.Cu") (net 8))
 (segment (start 184 55.75) (end 184 69.25) (width 0.4) (layer "F.Cu") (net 8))
 (segment (start 116.75 64.81) (end 116.75 72.77) (width 0.4) (layer "F.Cu") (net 8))
 (segment (start 157.66 114.75) (end 158.96 113.45) (width 0.4) (layer "F.Cu") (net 8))
 (segment (start 138.25 75) (end 141.18 77.93) (width 0.4) (layer "F.Cu") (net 8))
 (segment (start 147.04 34.25) (end 140.54 34.25) (width 0.4) (layer "F.Cu") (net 8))
 (segment (start 125.94 82) (end 125.94 78.82) (width 0.4) (layer "F.Cu") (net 8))
 (segment (start 173.399 45.149) (end 174.75 46.5) (width 0.4) (layer "F.Cu") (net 8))
 (segment (start 138.11 75.14) (end 138.25 75) (width 0.4) (layer "F.Cu") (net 8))
 (segment (start 129.25 34.2625) (end 128.25 35.2625) (width 0.4) (layer "F.Cu") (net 8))
 (segment (start 158.96 113.45) (end 158.96 107.4) (width 0.4) (layer "F.Cu") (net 8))
 (segment (start 129.76 75) (end 129.62 75.14) (width 0.4) (layer "F.Cu") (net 8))
 (segment (start 162.7775 34) (end 158.79 37.9875) (width 1.85) (layer "F.Cu") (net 4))
 (segment (start 171.17 34) (end 162.7775 34) (width 1.85) (layer "F.Cu") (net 4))
 (segment (start 106.25 59.39) (end 114.38 67.52) (width 0.4) (layer "F.Cu") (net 11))
 (segment (start 106.25 48.83) (end 106.25 59.39) (width 0.4) (layer "F.Cu") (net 11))
 (segment (start 108.25 45.75) (end 108.25 58.85) (width 0.4) (layer "F.Cu") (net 10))
 (segment (start 108.25 58.85) (end 114.38 64.98) (width 0.4) (layer "F.Cu") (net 10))
 (segment (start 106.25 43.75) (end 108.25 45.75) (width 0.4) (layer "F.Cu") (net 10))
 (segment (start 140.48 43.96) (end 114.38 70.06) (width 0.4) (layer "B.Cu") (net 7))
 (segment (start 186.2625 43.96) (end 140.48 43.96) (width 0.4) (layer "B.Cu") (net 7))
 (segment (start 185.3015 50.001) (end 156.796882 50.001) (width 0.4) (layer "B.Cu") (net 6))
 (segment (start 186.2625 49.04) (end 185.3015 50.001) (width 0.4) (layer "B.Cu") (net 6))
 (segment (start 130.216882 76.581) (end 118.361 76.581) (width 0.4) (layer "B.Cu") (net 6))
 (segment (start 156.796882 50.001) (end 130.216882 76.581) (width 0.4) (layer "B.Cu") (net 6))
 (segment (start 118.361 76.581) (end 114.38 72.6) (width 0.4) (layer "B.Cu") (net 6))
 (segment (start 143.72 107.4) (end 150.04 113.72) (width 0.4) (layer "F.Cu") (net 18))
 (segment (start 150.04 113.72) (end 150.04 114.75) (width 0.4) (layer "F.Cu") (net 18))
 (segment (start 134.8 88.32) (end 128.48 82) (width 0.4) (layer "B.Cu") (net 44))
 (segment (start 134.8 114.75) (end 134.8 88.32) (width 0.4) (layer "B.Cu") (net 44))
 (segment (start 152.58 103.56) (end 131.02 82) (width 0.4) (layer "F.Cu") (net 43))
 (segment (start 152.58 114.75) (end 152.58 103.56) (width 0.4) (layer "F.Cu") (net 43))
 (segment (start 144.96 113.72) (end 144.96 114.75) (width 0.4) (layer "F.Cu") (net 16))
 (segment (start 138.64 107.4) (end 144.96 113.72) (width 0.4) (layer "F.Cu") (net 16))
 (segment (start 147.5 113.72) (end 147.5 114.75) (width 0.4) (layer "F.Cu") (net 17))
 (segment (start 141.18 107.4) (end 147.5 113.72) (width 0.4) (layer "F.Cu") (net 17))
 (segment (start 133.56 107.4) (end 139.88 113.72) (width 0.4) (layer "F.Cu") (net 14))
 (segment (start 139.88 113.72) (end 139.88 114.75) (width 0.4) (layer "F.Cu") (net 14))
 (segment (start 136.1 107.4) (end 142.42 113.72) (width 0.4) (layer "F.Cu") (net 15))
 (segment (start 142.42 113.72) (end 142.42 114.75) (width 0.4) (layer "F.Cu") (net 15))
 (segment (start 131.02 107.4) (end 137.34 113.72) (width 0.4) (layer "F.Cu") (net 13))
 (segment (start 137.34 113.72) (end 137.34 114.75) (width 0.4) (layer "F.Cu") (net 13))
 (segment (start 120.25 54.03) (end 120.25 46.75) (width 0.5) (layer "F.Cu") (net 1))
 (segment (start 162.75 57) (end 154.5 48.75) (width 0.5) (layer "F.Cu") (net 1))
 (segment (start 111.75 103.75) (end 115.4 107.4) (width 0.5) (layer "F.Cu") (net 1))
 (segment (start 114.38 59.9) (end 120.25 54.03) (width 0.5) (layer "F.Cu") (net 1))
 (segment (start 115.4 107.4) (end 125.94 107.4) (width 0.5) (layer "F.Cu") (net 1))
 (segment (start 111.75 68.75) (end 111.75 103.75) (width 0.5) (layer "F.Cu") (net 1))
 (segment (start 154.5 48.75) (end 136.5 48.75) (width 0.5) (layer "F.Cu") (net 1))
 (segment (start 125.94 115.94) (end 125.94 107.4) (width 0.5) (layer "F.Cu") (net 1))
 (segment (start 131 121) (end 125.94 115.94) (width 0.5) (layer "F.Cu") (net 1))
 (segment (start 178.25 57) (end 162.75 57) (width 0.5) (layer "F.Cu") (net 1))
 (segment (start 136.5 48.75) (end 134.5 46.75) (width 0.5) (layer "F.Cu") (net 1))
 (segment (start 148.87 121) (end 131 121) (width 0.5) (layer "F.Cu") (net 1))
 (segment (start 155.12 114.75) (end 148.87 121) (width 0.5) (layer "F.Cu") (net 1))
 (via (at 111.75 68.75) (size 0.8) (drill 0.4) (layers "F.Cu" "B.Cu") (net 1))
 (segment (start 111.75 68.75) (end 111.75 62.53) (width 0.5) (layer "B.Cu") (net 1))
 (segment (start 120.319 46.8192) (end 120.25 46.75) (width 0.5) (layer "B.Cu") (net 1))
 (segment (start 120.25 46.75) (end 122.5 44.5) (width 0.5) (layer "B.Cu") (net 1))
 (segment (start 134.5 45.5) (end 134.5 46.75) (width 0.5) (layer "B.Cu") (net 1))
 (segment (start 122.5 44.5) (end 133.5 44.5) (width 0.5) (layer "B.Cu") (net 1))
 (segment (start 111.75 62.53) (end 114.38 59.9) (width 0.5) (layer "B.Cu") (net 1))
 (segment (start 133.5 44.5) (end 134.5 45.5) (width 0.5) (layer "B.Cu") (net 1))
 (segment (start 146.26 60.01) (end 146.26 63.01) (width 0.4) (layer "F.Cu") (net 39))
 (segment (start 140.54 38.75) (end 147.04 38.75) (width 0.4) (layer "F.Cu") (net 39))
 (segment (start 144.66 41.13) (end 144.66 46.75) (width 0.4) (layer "F.Cu") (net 39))
 (segment (start 147.04 38.75) (end 144.66 41.13) (width 0.4) (layer "F.Cu") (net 39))
 (segment (start 144.75 58.5) (end 146.26 60.01) (width 0.4) (layer "F.Cu") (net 39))
 (via (at 144.75 58.5) (size 0.8) (drill 0.4) (layers "F.Cu" "B.Cu") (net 39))
 (via (at 146.26 63.01) (size 0.8) (drill 0.4) (layers "F.Cu" "B.Cu") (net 39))
 (segment (start 146.26 63.01) (end 146.25 63) (width 0.4) (layer "B.Cu") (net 39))
 (segment (start 144.66 58.41) (end 144.75 58.5) (width 0.4) (layer "B.Cu") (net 39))
 (segment (start 146.26 82) (end 146.26 63.01) (width 0.4) (layer "B.Cu") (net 39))
 (segment (start 144.66 46.75) (end 144.66 58.41) (width 0.4) (layer "B.Cu") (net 39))
 (segment (start 130.41 46.75) (end 130.41 39.9225) (width 0.4) (layer "F.Cu") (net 2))
 (segment (start 143.72 66.03) (end 143.72 59.268) (width 0.4) (layer "F.Cu") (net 2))
 (segment (start 129.25 38.7625) (end 135.75 38.7625) (width 0.4) (layer "F.Cu") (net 2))
 (segment (start 130.41 39.9225) (end 129.25 38.7625) (width 0.4) (layer "F.Cu") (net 2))
 (segment (start 143.72 59.268) (end 131.202 46.75) (width 0.4) (layer "F.Cu") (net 2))
 (segment (start 131.202 46.75) (end 130.41 46.75) (width 0.4) (layer "F.Cu") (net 2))
 (via (at 143.72 66.03) (size 0.8) (drill 0.4) (layers "F.Cu" "B.Cu") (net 2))
 (via (at 143.72 66.03) (size 0.8) (drill 0.4) (layers "F.Cu" "B.Cu") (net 2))
 (segment (start 143.72 82) (end 143.72 66.03) (width 0.4) (layer "B.Cu") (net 2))
 (segment (start 126.75 53.25) (end 134.5 53.25) (width 1.85) (layer "F.Cu") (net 3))
 (segment (start 134.5 53.25) (end 138.25 57) (width 1.85) (layer "F.Cu") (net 3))
 (via (at 126.75 53.25) (size 0.8) (drill 0.4) (layers "F.Cu" "B.Cu") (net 3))
 (segment (start 120.626 31.874) (end 114.38 38.12) (width 1.85) (layer "B.Cu") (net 3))
 (segment (start 114.38 57.36) (end 122.64 57.36) (width 1.85) (layer "B.Cu") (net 3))
 (segment (start 173.71 34) (end 173.71 33.533381) (width 1.85) (layer "B.Cu") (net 3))
 (segment (start 173.71 33.533381) (end 172.050619 31.874) (width 1.85) (layer "B.Cu") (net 3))
 (segment (start 122.64 57.36) (end 126.75 53.25) (width 1.85) (layer "B.Cu") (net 3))
 (segment (start 114.38 38.12) (end 114.38 57.36) (width 1.85) (layer "B.Cu") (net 3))
 (segment (start 172.050619 31.874) (end 120.626 31.874) (width 1.85) (layer "B.Cu") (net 3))
 (segment (start 134 68.5) (end 134 73.25) (width 0.4) (layer "F.Cu") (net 40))
 (segment (start 134 73.25) (end 134.75 74) (width 0.4) (layer "F.Cu") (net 40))
 (via (at 134.75 74) (size 0.8) (drill 0.4) (layers "F.Cu" "B.Cu") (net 40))
 (via (at 134 68.5) (size 0.8) (drill 0.4) (layers "F.Cu" "B.Cu") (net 40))
 (segment (start 134.75 78.11) (end 138.64 82) (width 0.4) (layer "B.Cu") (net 40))
 (segment (start 134.75 74) (end 134.75 78.11) (width 0.4) (layer "B.Cu") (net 40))
 (segment (start 130.48 64.98) (end 134 68.5) (width 0.4) (layer "B.Cu") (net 40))
 (segment (start 129.62 64.98) (end 130.48 64.98) (width 0.4) (layer "B.Cu") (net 40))
 (segment (start 131.78 59.9) (end 129.62 59.9) (width 0.4) (layer "F.Cu") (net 36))
 (segment (start 153.88 82) (end 131.78 59.9) (width 0.4) (layer "F.Cu") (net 36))
 (segment (start 141.75 67.25) (end 131.86 57.36) (width 0.4) (layer "F.Cu") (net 19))
 (segment (start 131.86 57.36) (end 129.62 57.36) (width 0.4) (layer "F.Cu") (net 19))
 (via (at 141.75 67.25) (size 0.8) (drill 0.4) (layers "F.Cu" "B.Cu") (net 19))
 (segment (start 146.26 107.4) (end 142.5 103.64) (width 0.4) (layer "B.Cu") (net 19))
 (segment (start 142.5 103.64) (end 142.5 68) (width 0.4) (layer "B.Cu") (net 19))
 (segment (start 142.5 68) (end 141.75 67.25) (width 0.4) (layer "B.Cu") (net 19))
 (segment (start 131.779684 78.5) (end 128.5 78.5) (width 0.4) (layer "F.Cu") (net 20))
 (segment (start 125.15 72.6) (end 129.62 72.6) (width 0.4) (layer "F.Cu") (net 20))
 (segment (start 122.5 75.25) (end 125.15 72.6) (width 0.4) (layer "F.Cu") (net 20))
 (segment (start 134.776 81.496316) (end 131.779684 78.5) (width 0.4) (layer "F.Cu") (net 20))
 (segment (start 139.272316 87) (end 134.776 82.503684) (width 0.4) (layer "F.Cu") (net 20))
 (segment (start 134.776 82.503684) (end 134.776 81.496316) (width 0.4) (layer "F.Cu") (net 20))
 (segment (start 144.25 87) (end 139.272316 87) (width 0.4) (layer "F.Cu") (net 20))
 (segment (start 122.5 78.5) (end 122.5 75.25) (width 0.4) (layer "F.Cu") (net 20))
 (via (at 144.25 87) (size 0.8) (drill 0.4) (layers "F.Cu" "B.Cu") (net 20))
 (via (at 128.5 78.5) (size 0.8) (drill 0.4) (layers "F.Cu" "B.Cu") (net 20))
 (via (at 122.5 78.5) (size 0.8) (drill 0.4) (layers "F.Cu" "B.Cu") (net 20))
 (segment (start 148.8 107.4) (end 148.8 91.55) (width 0.4) (layer "B.Cu") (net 20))
 (segment (start 148.8 91.55) (end 144.25 87) (width 0.4) (layer "B.Cu") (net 20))
 (segment (start 128.5 78.5) (end 122.5 78.5) (width 0.4) (layer "B.Cu") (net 20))
 (segment (start 151.34 82) (end 131.78 62.44) (width 0.4) (layer "F.Cu") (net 37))
 (segment (start 131.78 62.44) (end 129.62 62.44) (width 0.4) (layer "F.Cu") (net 37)))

